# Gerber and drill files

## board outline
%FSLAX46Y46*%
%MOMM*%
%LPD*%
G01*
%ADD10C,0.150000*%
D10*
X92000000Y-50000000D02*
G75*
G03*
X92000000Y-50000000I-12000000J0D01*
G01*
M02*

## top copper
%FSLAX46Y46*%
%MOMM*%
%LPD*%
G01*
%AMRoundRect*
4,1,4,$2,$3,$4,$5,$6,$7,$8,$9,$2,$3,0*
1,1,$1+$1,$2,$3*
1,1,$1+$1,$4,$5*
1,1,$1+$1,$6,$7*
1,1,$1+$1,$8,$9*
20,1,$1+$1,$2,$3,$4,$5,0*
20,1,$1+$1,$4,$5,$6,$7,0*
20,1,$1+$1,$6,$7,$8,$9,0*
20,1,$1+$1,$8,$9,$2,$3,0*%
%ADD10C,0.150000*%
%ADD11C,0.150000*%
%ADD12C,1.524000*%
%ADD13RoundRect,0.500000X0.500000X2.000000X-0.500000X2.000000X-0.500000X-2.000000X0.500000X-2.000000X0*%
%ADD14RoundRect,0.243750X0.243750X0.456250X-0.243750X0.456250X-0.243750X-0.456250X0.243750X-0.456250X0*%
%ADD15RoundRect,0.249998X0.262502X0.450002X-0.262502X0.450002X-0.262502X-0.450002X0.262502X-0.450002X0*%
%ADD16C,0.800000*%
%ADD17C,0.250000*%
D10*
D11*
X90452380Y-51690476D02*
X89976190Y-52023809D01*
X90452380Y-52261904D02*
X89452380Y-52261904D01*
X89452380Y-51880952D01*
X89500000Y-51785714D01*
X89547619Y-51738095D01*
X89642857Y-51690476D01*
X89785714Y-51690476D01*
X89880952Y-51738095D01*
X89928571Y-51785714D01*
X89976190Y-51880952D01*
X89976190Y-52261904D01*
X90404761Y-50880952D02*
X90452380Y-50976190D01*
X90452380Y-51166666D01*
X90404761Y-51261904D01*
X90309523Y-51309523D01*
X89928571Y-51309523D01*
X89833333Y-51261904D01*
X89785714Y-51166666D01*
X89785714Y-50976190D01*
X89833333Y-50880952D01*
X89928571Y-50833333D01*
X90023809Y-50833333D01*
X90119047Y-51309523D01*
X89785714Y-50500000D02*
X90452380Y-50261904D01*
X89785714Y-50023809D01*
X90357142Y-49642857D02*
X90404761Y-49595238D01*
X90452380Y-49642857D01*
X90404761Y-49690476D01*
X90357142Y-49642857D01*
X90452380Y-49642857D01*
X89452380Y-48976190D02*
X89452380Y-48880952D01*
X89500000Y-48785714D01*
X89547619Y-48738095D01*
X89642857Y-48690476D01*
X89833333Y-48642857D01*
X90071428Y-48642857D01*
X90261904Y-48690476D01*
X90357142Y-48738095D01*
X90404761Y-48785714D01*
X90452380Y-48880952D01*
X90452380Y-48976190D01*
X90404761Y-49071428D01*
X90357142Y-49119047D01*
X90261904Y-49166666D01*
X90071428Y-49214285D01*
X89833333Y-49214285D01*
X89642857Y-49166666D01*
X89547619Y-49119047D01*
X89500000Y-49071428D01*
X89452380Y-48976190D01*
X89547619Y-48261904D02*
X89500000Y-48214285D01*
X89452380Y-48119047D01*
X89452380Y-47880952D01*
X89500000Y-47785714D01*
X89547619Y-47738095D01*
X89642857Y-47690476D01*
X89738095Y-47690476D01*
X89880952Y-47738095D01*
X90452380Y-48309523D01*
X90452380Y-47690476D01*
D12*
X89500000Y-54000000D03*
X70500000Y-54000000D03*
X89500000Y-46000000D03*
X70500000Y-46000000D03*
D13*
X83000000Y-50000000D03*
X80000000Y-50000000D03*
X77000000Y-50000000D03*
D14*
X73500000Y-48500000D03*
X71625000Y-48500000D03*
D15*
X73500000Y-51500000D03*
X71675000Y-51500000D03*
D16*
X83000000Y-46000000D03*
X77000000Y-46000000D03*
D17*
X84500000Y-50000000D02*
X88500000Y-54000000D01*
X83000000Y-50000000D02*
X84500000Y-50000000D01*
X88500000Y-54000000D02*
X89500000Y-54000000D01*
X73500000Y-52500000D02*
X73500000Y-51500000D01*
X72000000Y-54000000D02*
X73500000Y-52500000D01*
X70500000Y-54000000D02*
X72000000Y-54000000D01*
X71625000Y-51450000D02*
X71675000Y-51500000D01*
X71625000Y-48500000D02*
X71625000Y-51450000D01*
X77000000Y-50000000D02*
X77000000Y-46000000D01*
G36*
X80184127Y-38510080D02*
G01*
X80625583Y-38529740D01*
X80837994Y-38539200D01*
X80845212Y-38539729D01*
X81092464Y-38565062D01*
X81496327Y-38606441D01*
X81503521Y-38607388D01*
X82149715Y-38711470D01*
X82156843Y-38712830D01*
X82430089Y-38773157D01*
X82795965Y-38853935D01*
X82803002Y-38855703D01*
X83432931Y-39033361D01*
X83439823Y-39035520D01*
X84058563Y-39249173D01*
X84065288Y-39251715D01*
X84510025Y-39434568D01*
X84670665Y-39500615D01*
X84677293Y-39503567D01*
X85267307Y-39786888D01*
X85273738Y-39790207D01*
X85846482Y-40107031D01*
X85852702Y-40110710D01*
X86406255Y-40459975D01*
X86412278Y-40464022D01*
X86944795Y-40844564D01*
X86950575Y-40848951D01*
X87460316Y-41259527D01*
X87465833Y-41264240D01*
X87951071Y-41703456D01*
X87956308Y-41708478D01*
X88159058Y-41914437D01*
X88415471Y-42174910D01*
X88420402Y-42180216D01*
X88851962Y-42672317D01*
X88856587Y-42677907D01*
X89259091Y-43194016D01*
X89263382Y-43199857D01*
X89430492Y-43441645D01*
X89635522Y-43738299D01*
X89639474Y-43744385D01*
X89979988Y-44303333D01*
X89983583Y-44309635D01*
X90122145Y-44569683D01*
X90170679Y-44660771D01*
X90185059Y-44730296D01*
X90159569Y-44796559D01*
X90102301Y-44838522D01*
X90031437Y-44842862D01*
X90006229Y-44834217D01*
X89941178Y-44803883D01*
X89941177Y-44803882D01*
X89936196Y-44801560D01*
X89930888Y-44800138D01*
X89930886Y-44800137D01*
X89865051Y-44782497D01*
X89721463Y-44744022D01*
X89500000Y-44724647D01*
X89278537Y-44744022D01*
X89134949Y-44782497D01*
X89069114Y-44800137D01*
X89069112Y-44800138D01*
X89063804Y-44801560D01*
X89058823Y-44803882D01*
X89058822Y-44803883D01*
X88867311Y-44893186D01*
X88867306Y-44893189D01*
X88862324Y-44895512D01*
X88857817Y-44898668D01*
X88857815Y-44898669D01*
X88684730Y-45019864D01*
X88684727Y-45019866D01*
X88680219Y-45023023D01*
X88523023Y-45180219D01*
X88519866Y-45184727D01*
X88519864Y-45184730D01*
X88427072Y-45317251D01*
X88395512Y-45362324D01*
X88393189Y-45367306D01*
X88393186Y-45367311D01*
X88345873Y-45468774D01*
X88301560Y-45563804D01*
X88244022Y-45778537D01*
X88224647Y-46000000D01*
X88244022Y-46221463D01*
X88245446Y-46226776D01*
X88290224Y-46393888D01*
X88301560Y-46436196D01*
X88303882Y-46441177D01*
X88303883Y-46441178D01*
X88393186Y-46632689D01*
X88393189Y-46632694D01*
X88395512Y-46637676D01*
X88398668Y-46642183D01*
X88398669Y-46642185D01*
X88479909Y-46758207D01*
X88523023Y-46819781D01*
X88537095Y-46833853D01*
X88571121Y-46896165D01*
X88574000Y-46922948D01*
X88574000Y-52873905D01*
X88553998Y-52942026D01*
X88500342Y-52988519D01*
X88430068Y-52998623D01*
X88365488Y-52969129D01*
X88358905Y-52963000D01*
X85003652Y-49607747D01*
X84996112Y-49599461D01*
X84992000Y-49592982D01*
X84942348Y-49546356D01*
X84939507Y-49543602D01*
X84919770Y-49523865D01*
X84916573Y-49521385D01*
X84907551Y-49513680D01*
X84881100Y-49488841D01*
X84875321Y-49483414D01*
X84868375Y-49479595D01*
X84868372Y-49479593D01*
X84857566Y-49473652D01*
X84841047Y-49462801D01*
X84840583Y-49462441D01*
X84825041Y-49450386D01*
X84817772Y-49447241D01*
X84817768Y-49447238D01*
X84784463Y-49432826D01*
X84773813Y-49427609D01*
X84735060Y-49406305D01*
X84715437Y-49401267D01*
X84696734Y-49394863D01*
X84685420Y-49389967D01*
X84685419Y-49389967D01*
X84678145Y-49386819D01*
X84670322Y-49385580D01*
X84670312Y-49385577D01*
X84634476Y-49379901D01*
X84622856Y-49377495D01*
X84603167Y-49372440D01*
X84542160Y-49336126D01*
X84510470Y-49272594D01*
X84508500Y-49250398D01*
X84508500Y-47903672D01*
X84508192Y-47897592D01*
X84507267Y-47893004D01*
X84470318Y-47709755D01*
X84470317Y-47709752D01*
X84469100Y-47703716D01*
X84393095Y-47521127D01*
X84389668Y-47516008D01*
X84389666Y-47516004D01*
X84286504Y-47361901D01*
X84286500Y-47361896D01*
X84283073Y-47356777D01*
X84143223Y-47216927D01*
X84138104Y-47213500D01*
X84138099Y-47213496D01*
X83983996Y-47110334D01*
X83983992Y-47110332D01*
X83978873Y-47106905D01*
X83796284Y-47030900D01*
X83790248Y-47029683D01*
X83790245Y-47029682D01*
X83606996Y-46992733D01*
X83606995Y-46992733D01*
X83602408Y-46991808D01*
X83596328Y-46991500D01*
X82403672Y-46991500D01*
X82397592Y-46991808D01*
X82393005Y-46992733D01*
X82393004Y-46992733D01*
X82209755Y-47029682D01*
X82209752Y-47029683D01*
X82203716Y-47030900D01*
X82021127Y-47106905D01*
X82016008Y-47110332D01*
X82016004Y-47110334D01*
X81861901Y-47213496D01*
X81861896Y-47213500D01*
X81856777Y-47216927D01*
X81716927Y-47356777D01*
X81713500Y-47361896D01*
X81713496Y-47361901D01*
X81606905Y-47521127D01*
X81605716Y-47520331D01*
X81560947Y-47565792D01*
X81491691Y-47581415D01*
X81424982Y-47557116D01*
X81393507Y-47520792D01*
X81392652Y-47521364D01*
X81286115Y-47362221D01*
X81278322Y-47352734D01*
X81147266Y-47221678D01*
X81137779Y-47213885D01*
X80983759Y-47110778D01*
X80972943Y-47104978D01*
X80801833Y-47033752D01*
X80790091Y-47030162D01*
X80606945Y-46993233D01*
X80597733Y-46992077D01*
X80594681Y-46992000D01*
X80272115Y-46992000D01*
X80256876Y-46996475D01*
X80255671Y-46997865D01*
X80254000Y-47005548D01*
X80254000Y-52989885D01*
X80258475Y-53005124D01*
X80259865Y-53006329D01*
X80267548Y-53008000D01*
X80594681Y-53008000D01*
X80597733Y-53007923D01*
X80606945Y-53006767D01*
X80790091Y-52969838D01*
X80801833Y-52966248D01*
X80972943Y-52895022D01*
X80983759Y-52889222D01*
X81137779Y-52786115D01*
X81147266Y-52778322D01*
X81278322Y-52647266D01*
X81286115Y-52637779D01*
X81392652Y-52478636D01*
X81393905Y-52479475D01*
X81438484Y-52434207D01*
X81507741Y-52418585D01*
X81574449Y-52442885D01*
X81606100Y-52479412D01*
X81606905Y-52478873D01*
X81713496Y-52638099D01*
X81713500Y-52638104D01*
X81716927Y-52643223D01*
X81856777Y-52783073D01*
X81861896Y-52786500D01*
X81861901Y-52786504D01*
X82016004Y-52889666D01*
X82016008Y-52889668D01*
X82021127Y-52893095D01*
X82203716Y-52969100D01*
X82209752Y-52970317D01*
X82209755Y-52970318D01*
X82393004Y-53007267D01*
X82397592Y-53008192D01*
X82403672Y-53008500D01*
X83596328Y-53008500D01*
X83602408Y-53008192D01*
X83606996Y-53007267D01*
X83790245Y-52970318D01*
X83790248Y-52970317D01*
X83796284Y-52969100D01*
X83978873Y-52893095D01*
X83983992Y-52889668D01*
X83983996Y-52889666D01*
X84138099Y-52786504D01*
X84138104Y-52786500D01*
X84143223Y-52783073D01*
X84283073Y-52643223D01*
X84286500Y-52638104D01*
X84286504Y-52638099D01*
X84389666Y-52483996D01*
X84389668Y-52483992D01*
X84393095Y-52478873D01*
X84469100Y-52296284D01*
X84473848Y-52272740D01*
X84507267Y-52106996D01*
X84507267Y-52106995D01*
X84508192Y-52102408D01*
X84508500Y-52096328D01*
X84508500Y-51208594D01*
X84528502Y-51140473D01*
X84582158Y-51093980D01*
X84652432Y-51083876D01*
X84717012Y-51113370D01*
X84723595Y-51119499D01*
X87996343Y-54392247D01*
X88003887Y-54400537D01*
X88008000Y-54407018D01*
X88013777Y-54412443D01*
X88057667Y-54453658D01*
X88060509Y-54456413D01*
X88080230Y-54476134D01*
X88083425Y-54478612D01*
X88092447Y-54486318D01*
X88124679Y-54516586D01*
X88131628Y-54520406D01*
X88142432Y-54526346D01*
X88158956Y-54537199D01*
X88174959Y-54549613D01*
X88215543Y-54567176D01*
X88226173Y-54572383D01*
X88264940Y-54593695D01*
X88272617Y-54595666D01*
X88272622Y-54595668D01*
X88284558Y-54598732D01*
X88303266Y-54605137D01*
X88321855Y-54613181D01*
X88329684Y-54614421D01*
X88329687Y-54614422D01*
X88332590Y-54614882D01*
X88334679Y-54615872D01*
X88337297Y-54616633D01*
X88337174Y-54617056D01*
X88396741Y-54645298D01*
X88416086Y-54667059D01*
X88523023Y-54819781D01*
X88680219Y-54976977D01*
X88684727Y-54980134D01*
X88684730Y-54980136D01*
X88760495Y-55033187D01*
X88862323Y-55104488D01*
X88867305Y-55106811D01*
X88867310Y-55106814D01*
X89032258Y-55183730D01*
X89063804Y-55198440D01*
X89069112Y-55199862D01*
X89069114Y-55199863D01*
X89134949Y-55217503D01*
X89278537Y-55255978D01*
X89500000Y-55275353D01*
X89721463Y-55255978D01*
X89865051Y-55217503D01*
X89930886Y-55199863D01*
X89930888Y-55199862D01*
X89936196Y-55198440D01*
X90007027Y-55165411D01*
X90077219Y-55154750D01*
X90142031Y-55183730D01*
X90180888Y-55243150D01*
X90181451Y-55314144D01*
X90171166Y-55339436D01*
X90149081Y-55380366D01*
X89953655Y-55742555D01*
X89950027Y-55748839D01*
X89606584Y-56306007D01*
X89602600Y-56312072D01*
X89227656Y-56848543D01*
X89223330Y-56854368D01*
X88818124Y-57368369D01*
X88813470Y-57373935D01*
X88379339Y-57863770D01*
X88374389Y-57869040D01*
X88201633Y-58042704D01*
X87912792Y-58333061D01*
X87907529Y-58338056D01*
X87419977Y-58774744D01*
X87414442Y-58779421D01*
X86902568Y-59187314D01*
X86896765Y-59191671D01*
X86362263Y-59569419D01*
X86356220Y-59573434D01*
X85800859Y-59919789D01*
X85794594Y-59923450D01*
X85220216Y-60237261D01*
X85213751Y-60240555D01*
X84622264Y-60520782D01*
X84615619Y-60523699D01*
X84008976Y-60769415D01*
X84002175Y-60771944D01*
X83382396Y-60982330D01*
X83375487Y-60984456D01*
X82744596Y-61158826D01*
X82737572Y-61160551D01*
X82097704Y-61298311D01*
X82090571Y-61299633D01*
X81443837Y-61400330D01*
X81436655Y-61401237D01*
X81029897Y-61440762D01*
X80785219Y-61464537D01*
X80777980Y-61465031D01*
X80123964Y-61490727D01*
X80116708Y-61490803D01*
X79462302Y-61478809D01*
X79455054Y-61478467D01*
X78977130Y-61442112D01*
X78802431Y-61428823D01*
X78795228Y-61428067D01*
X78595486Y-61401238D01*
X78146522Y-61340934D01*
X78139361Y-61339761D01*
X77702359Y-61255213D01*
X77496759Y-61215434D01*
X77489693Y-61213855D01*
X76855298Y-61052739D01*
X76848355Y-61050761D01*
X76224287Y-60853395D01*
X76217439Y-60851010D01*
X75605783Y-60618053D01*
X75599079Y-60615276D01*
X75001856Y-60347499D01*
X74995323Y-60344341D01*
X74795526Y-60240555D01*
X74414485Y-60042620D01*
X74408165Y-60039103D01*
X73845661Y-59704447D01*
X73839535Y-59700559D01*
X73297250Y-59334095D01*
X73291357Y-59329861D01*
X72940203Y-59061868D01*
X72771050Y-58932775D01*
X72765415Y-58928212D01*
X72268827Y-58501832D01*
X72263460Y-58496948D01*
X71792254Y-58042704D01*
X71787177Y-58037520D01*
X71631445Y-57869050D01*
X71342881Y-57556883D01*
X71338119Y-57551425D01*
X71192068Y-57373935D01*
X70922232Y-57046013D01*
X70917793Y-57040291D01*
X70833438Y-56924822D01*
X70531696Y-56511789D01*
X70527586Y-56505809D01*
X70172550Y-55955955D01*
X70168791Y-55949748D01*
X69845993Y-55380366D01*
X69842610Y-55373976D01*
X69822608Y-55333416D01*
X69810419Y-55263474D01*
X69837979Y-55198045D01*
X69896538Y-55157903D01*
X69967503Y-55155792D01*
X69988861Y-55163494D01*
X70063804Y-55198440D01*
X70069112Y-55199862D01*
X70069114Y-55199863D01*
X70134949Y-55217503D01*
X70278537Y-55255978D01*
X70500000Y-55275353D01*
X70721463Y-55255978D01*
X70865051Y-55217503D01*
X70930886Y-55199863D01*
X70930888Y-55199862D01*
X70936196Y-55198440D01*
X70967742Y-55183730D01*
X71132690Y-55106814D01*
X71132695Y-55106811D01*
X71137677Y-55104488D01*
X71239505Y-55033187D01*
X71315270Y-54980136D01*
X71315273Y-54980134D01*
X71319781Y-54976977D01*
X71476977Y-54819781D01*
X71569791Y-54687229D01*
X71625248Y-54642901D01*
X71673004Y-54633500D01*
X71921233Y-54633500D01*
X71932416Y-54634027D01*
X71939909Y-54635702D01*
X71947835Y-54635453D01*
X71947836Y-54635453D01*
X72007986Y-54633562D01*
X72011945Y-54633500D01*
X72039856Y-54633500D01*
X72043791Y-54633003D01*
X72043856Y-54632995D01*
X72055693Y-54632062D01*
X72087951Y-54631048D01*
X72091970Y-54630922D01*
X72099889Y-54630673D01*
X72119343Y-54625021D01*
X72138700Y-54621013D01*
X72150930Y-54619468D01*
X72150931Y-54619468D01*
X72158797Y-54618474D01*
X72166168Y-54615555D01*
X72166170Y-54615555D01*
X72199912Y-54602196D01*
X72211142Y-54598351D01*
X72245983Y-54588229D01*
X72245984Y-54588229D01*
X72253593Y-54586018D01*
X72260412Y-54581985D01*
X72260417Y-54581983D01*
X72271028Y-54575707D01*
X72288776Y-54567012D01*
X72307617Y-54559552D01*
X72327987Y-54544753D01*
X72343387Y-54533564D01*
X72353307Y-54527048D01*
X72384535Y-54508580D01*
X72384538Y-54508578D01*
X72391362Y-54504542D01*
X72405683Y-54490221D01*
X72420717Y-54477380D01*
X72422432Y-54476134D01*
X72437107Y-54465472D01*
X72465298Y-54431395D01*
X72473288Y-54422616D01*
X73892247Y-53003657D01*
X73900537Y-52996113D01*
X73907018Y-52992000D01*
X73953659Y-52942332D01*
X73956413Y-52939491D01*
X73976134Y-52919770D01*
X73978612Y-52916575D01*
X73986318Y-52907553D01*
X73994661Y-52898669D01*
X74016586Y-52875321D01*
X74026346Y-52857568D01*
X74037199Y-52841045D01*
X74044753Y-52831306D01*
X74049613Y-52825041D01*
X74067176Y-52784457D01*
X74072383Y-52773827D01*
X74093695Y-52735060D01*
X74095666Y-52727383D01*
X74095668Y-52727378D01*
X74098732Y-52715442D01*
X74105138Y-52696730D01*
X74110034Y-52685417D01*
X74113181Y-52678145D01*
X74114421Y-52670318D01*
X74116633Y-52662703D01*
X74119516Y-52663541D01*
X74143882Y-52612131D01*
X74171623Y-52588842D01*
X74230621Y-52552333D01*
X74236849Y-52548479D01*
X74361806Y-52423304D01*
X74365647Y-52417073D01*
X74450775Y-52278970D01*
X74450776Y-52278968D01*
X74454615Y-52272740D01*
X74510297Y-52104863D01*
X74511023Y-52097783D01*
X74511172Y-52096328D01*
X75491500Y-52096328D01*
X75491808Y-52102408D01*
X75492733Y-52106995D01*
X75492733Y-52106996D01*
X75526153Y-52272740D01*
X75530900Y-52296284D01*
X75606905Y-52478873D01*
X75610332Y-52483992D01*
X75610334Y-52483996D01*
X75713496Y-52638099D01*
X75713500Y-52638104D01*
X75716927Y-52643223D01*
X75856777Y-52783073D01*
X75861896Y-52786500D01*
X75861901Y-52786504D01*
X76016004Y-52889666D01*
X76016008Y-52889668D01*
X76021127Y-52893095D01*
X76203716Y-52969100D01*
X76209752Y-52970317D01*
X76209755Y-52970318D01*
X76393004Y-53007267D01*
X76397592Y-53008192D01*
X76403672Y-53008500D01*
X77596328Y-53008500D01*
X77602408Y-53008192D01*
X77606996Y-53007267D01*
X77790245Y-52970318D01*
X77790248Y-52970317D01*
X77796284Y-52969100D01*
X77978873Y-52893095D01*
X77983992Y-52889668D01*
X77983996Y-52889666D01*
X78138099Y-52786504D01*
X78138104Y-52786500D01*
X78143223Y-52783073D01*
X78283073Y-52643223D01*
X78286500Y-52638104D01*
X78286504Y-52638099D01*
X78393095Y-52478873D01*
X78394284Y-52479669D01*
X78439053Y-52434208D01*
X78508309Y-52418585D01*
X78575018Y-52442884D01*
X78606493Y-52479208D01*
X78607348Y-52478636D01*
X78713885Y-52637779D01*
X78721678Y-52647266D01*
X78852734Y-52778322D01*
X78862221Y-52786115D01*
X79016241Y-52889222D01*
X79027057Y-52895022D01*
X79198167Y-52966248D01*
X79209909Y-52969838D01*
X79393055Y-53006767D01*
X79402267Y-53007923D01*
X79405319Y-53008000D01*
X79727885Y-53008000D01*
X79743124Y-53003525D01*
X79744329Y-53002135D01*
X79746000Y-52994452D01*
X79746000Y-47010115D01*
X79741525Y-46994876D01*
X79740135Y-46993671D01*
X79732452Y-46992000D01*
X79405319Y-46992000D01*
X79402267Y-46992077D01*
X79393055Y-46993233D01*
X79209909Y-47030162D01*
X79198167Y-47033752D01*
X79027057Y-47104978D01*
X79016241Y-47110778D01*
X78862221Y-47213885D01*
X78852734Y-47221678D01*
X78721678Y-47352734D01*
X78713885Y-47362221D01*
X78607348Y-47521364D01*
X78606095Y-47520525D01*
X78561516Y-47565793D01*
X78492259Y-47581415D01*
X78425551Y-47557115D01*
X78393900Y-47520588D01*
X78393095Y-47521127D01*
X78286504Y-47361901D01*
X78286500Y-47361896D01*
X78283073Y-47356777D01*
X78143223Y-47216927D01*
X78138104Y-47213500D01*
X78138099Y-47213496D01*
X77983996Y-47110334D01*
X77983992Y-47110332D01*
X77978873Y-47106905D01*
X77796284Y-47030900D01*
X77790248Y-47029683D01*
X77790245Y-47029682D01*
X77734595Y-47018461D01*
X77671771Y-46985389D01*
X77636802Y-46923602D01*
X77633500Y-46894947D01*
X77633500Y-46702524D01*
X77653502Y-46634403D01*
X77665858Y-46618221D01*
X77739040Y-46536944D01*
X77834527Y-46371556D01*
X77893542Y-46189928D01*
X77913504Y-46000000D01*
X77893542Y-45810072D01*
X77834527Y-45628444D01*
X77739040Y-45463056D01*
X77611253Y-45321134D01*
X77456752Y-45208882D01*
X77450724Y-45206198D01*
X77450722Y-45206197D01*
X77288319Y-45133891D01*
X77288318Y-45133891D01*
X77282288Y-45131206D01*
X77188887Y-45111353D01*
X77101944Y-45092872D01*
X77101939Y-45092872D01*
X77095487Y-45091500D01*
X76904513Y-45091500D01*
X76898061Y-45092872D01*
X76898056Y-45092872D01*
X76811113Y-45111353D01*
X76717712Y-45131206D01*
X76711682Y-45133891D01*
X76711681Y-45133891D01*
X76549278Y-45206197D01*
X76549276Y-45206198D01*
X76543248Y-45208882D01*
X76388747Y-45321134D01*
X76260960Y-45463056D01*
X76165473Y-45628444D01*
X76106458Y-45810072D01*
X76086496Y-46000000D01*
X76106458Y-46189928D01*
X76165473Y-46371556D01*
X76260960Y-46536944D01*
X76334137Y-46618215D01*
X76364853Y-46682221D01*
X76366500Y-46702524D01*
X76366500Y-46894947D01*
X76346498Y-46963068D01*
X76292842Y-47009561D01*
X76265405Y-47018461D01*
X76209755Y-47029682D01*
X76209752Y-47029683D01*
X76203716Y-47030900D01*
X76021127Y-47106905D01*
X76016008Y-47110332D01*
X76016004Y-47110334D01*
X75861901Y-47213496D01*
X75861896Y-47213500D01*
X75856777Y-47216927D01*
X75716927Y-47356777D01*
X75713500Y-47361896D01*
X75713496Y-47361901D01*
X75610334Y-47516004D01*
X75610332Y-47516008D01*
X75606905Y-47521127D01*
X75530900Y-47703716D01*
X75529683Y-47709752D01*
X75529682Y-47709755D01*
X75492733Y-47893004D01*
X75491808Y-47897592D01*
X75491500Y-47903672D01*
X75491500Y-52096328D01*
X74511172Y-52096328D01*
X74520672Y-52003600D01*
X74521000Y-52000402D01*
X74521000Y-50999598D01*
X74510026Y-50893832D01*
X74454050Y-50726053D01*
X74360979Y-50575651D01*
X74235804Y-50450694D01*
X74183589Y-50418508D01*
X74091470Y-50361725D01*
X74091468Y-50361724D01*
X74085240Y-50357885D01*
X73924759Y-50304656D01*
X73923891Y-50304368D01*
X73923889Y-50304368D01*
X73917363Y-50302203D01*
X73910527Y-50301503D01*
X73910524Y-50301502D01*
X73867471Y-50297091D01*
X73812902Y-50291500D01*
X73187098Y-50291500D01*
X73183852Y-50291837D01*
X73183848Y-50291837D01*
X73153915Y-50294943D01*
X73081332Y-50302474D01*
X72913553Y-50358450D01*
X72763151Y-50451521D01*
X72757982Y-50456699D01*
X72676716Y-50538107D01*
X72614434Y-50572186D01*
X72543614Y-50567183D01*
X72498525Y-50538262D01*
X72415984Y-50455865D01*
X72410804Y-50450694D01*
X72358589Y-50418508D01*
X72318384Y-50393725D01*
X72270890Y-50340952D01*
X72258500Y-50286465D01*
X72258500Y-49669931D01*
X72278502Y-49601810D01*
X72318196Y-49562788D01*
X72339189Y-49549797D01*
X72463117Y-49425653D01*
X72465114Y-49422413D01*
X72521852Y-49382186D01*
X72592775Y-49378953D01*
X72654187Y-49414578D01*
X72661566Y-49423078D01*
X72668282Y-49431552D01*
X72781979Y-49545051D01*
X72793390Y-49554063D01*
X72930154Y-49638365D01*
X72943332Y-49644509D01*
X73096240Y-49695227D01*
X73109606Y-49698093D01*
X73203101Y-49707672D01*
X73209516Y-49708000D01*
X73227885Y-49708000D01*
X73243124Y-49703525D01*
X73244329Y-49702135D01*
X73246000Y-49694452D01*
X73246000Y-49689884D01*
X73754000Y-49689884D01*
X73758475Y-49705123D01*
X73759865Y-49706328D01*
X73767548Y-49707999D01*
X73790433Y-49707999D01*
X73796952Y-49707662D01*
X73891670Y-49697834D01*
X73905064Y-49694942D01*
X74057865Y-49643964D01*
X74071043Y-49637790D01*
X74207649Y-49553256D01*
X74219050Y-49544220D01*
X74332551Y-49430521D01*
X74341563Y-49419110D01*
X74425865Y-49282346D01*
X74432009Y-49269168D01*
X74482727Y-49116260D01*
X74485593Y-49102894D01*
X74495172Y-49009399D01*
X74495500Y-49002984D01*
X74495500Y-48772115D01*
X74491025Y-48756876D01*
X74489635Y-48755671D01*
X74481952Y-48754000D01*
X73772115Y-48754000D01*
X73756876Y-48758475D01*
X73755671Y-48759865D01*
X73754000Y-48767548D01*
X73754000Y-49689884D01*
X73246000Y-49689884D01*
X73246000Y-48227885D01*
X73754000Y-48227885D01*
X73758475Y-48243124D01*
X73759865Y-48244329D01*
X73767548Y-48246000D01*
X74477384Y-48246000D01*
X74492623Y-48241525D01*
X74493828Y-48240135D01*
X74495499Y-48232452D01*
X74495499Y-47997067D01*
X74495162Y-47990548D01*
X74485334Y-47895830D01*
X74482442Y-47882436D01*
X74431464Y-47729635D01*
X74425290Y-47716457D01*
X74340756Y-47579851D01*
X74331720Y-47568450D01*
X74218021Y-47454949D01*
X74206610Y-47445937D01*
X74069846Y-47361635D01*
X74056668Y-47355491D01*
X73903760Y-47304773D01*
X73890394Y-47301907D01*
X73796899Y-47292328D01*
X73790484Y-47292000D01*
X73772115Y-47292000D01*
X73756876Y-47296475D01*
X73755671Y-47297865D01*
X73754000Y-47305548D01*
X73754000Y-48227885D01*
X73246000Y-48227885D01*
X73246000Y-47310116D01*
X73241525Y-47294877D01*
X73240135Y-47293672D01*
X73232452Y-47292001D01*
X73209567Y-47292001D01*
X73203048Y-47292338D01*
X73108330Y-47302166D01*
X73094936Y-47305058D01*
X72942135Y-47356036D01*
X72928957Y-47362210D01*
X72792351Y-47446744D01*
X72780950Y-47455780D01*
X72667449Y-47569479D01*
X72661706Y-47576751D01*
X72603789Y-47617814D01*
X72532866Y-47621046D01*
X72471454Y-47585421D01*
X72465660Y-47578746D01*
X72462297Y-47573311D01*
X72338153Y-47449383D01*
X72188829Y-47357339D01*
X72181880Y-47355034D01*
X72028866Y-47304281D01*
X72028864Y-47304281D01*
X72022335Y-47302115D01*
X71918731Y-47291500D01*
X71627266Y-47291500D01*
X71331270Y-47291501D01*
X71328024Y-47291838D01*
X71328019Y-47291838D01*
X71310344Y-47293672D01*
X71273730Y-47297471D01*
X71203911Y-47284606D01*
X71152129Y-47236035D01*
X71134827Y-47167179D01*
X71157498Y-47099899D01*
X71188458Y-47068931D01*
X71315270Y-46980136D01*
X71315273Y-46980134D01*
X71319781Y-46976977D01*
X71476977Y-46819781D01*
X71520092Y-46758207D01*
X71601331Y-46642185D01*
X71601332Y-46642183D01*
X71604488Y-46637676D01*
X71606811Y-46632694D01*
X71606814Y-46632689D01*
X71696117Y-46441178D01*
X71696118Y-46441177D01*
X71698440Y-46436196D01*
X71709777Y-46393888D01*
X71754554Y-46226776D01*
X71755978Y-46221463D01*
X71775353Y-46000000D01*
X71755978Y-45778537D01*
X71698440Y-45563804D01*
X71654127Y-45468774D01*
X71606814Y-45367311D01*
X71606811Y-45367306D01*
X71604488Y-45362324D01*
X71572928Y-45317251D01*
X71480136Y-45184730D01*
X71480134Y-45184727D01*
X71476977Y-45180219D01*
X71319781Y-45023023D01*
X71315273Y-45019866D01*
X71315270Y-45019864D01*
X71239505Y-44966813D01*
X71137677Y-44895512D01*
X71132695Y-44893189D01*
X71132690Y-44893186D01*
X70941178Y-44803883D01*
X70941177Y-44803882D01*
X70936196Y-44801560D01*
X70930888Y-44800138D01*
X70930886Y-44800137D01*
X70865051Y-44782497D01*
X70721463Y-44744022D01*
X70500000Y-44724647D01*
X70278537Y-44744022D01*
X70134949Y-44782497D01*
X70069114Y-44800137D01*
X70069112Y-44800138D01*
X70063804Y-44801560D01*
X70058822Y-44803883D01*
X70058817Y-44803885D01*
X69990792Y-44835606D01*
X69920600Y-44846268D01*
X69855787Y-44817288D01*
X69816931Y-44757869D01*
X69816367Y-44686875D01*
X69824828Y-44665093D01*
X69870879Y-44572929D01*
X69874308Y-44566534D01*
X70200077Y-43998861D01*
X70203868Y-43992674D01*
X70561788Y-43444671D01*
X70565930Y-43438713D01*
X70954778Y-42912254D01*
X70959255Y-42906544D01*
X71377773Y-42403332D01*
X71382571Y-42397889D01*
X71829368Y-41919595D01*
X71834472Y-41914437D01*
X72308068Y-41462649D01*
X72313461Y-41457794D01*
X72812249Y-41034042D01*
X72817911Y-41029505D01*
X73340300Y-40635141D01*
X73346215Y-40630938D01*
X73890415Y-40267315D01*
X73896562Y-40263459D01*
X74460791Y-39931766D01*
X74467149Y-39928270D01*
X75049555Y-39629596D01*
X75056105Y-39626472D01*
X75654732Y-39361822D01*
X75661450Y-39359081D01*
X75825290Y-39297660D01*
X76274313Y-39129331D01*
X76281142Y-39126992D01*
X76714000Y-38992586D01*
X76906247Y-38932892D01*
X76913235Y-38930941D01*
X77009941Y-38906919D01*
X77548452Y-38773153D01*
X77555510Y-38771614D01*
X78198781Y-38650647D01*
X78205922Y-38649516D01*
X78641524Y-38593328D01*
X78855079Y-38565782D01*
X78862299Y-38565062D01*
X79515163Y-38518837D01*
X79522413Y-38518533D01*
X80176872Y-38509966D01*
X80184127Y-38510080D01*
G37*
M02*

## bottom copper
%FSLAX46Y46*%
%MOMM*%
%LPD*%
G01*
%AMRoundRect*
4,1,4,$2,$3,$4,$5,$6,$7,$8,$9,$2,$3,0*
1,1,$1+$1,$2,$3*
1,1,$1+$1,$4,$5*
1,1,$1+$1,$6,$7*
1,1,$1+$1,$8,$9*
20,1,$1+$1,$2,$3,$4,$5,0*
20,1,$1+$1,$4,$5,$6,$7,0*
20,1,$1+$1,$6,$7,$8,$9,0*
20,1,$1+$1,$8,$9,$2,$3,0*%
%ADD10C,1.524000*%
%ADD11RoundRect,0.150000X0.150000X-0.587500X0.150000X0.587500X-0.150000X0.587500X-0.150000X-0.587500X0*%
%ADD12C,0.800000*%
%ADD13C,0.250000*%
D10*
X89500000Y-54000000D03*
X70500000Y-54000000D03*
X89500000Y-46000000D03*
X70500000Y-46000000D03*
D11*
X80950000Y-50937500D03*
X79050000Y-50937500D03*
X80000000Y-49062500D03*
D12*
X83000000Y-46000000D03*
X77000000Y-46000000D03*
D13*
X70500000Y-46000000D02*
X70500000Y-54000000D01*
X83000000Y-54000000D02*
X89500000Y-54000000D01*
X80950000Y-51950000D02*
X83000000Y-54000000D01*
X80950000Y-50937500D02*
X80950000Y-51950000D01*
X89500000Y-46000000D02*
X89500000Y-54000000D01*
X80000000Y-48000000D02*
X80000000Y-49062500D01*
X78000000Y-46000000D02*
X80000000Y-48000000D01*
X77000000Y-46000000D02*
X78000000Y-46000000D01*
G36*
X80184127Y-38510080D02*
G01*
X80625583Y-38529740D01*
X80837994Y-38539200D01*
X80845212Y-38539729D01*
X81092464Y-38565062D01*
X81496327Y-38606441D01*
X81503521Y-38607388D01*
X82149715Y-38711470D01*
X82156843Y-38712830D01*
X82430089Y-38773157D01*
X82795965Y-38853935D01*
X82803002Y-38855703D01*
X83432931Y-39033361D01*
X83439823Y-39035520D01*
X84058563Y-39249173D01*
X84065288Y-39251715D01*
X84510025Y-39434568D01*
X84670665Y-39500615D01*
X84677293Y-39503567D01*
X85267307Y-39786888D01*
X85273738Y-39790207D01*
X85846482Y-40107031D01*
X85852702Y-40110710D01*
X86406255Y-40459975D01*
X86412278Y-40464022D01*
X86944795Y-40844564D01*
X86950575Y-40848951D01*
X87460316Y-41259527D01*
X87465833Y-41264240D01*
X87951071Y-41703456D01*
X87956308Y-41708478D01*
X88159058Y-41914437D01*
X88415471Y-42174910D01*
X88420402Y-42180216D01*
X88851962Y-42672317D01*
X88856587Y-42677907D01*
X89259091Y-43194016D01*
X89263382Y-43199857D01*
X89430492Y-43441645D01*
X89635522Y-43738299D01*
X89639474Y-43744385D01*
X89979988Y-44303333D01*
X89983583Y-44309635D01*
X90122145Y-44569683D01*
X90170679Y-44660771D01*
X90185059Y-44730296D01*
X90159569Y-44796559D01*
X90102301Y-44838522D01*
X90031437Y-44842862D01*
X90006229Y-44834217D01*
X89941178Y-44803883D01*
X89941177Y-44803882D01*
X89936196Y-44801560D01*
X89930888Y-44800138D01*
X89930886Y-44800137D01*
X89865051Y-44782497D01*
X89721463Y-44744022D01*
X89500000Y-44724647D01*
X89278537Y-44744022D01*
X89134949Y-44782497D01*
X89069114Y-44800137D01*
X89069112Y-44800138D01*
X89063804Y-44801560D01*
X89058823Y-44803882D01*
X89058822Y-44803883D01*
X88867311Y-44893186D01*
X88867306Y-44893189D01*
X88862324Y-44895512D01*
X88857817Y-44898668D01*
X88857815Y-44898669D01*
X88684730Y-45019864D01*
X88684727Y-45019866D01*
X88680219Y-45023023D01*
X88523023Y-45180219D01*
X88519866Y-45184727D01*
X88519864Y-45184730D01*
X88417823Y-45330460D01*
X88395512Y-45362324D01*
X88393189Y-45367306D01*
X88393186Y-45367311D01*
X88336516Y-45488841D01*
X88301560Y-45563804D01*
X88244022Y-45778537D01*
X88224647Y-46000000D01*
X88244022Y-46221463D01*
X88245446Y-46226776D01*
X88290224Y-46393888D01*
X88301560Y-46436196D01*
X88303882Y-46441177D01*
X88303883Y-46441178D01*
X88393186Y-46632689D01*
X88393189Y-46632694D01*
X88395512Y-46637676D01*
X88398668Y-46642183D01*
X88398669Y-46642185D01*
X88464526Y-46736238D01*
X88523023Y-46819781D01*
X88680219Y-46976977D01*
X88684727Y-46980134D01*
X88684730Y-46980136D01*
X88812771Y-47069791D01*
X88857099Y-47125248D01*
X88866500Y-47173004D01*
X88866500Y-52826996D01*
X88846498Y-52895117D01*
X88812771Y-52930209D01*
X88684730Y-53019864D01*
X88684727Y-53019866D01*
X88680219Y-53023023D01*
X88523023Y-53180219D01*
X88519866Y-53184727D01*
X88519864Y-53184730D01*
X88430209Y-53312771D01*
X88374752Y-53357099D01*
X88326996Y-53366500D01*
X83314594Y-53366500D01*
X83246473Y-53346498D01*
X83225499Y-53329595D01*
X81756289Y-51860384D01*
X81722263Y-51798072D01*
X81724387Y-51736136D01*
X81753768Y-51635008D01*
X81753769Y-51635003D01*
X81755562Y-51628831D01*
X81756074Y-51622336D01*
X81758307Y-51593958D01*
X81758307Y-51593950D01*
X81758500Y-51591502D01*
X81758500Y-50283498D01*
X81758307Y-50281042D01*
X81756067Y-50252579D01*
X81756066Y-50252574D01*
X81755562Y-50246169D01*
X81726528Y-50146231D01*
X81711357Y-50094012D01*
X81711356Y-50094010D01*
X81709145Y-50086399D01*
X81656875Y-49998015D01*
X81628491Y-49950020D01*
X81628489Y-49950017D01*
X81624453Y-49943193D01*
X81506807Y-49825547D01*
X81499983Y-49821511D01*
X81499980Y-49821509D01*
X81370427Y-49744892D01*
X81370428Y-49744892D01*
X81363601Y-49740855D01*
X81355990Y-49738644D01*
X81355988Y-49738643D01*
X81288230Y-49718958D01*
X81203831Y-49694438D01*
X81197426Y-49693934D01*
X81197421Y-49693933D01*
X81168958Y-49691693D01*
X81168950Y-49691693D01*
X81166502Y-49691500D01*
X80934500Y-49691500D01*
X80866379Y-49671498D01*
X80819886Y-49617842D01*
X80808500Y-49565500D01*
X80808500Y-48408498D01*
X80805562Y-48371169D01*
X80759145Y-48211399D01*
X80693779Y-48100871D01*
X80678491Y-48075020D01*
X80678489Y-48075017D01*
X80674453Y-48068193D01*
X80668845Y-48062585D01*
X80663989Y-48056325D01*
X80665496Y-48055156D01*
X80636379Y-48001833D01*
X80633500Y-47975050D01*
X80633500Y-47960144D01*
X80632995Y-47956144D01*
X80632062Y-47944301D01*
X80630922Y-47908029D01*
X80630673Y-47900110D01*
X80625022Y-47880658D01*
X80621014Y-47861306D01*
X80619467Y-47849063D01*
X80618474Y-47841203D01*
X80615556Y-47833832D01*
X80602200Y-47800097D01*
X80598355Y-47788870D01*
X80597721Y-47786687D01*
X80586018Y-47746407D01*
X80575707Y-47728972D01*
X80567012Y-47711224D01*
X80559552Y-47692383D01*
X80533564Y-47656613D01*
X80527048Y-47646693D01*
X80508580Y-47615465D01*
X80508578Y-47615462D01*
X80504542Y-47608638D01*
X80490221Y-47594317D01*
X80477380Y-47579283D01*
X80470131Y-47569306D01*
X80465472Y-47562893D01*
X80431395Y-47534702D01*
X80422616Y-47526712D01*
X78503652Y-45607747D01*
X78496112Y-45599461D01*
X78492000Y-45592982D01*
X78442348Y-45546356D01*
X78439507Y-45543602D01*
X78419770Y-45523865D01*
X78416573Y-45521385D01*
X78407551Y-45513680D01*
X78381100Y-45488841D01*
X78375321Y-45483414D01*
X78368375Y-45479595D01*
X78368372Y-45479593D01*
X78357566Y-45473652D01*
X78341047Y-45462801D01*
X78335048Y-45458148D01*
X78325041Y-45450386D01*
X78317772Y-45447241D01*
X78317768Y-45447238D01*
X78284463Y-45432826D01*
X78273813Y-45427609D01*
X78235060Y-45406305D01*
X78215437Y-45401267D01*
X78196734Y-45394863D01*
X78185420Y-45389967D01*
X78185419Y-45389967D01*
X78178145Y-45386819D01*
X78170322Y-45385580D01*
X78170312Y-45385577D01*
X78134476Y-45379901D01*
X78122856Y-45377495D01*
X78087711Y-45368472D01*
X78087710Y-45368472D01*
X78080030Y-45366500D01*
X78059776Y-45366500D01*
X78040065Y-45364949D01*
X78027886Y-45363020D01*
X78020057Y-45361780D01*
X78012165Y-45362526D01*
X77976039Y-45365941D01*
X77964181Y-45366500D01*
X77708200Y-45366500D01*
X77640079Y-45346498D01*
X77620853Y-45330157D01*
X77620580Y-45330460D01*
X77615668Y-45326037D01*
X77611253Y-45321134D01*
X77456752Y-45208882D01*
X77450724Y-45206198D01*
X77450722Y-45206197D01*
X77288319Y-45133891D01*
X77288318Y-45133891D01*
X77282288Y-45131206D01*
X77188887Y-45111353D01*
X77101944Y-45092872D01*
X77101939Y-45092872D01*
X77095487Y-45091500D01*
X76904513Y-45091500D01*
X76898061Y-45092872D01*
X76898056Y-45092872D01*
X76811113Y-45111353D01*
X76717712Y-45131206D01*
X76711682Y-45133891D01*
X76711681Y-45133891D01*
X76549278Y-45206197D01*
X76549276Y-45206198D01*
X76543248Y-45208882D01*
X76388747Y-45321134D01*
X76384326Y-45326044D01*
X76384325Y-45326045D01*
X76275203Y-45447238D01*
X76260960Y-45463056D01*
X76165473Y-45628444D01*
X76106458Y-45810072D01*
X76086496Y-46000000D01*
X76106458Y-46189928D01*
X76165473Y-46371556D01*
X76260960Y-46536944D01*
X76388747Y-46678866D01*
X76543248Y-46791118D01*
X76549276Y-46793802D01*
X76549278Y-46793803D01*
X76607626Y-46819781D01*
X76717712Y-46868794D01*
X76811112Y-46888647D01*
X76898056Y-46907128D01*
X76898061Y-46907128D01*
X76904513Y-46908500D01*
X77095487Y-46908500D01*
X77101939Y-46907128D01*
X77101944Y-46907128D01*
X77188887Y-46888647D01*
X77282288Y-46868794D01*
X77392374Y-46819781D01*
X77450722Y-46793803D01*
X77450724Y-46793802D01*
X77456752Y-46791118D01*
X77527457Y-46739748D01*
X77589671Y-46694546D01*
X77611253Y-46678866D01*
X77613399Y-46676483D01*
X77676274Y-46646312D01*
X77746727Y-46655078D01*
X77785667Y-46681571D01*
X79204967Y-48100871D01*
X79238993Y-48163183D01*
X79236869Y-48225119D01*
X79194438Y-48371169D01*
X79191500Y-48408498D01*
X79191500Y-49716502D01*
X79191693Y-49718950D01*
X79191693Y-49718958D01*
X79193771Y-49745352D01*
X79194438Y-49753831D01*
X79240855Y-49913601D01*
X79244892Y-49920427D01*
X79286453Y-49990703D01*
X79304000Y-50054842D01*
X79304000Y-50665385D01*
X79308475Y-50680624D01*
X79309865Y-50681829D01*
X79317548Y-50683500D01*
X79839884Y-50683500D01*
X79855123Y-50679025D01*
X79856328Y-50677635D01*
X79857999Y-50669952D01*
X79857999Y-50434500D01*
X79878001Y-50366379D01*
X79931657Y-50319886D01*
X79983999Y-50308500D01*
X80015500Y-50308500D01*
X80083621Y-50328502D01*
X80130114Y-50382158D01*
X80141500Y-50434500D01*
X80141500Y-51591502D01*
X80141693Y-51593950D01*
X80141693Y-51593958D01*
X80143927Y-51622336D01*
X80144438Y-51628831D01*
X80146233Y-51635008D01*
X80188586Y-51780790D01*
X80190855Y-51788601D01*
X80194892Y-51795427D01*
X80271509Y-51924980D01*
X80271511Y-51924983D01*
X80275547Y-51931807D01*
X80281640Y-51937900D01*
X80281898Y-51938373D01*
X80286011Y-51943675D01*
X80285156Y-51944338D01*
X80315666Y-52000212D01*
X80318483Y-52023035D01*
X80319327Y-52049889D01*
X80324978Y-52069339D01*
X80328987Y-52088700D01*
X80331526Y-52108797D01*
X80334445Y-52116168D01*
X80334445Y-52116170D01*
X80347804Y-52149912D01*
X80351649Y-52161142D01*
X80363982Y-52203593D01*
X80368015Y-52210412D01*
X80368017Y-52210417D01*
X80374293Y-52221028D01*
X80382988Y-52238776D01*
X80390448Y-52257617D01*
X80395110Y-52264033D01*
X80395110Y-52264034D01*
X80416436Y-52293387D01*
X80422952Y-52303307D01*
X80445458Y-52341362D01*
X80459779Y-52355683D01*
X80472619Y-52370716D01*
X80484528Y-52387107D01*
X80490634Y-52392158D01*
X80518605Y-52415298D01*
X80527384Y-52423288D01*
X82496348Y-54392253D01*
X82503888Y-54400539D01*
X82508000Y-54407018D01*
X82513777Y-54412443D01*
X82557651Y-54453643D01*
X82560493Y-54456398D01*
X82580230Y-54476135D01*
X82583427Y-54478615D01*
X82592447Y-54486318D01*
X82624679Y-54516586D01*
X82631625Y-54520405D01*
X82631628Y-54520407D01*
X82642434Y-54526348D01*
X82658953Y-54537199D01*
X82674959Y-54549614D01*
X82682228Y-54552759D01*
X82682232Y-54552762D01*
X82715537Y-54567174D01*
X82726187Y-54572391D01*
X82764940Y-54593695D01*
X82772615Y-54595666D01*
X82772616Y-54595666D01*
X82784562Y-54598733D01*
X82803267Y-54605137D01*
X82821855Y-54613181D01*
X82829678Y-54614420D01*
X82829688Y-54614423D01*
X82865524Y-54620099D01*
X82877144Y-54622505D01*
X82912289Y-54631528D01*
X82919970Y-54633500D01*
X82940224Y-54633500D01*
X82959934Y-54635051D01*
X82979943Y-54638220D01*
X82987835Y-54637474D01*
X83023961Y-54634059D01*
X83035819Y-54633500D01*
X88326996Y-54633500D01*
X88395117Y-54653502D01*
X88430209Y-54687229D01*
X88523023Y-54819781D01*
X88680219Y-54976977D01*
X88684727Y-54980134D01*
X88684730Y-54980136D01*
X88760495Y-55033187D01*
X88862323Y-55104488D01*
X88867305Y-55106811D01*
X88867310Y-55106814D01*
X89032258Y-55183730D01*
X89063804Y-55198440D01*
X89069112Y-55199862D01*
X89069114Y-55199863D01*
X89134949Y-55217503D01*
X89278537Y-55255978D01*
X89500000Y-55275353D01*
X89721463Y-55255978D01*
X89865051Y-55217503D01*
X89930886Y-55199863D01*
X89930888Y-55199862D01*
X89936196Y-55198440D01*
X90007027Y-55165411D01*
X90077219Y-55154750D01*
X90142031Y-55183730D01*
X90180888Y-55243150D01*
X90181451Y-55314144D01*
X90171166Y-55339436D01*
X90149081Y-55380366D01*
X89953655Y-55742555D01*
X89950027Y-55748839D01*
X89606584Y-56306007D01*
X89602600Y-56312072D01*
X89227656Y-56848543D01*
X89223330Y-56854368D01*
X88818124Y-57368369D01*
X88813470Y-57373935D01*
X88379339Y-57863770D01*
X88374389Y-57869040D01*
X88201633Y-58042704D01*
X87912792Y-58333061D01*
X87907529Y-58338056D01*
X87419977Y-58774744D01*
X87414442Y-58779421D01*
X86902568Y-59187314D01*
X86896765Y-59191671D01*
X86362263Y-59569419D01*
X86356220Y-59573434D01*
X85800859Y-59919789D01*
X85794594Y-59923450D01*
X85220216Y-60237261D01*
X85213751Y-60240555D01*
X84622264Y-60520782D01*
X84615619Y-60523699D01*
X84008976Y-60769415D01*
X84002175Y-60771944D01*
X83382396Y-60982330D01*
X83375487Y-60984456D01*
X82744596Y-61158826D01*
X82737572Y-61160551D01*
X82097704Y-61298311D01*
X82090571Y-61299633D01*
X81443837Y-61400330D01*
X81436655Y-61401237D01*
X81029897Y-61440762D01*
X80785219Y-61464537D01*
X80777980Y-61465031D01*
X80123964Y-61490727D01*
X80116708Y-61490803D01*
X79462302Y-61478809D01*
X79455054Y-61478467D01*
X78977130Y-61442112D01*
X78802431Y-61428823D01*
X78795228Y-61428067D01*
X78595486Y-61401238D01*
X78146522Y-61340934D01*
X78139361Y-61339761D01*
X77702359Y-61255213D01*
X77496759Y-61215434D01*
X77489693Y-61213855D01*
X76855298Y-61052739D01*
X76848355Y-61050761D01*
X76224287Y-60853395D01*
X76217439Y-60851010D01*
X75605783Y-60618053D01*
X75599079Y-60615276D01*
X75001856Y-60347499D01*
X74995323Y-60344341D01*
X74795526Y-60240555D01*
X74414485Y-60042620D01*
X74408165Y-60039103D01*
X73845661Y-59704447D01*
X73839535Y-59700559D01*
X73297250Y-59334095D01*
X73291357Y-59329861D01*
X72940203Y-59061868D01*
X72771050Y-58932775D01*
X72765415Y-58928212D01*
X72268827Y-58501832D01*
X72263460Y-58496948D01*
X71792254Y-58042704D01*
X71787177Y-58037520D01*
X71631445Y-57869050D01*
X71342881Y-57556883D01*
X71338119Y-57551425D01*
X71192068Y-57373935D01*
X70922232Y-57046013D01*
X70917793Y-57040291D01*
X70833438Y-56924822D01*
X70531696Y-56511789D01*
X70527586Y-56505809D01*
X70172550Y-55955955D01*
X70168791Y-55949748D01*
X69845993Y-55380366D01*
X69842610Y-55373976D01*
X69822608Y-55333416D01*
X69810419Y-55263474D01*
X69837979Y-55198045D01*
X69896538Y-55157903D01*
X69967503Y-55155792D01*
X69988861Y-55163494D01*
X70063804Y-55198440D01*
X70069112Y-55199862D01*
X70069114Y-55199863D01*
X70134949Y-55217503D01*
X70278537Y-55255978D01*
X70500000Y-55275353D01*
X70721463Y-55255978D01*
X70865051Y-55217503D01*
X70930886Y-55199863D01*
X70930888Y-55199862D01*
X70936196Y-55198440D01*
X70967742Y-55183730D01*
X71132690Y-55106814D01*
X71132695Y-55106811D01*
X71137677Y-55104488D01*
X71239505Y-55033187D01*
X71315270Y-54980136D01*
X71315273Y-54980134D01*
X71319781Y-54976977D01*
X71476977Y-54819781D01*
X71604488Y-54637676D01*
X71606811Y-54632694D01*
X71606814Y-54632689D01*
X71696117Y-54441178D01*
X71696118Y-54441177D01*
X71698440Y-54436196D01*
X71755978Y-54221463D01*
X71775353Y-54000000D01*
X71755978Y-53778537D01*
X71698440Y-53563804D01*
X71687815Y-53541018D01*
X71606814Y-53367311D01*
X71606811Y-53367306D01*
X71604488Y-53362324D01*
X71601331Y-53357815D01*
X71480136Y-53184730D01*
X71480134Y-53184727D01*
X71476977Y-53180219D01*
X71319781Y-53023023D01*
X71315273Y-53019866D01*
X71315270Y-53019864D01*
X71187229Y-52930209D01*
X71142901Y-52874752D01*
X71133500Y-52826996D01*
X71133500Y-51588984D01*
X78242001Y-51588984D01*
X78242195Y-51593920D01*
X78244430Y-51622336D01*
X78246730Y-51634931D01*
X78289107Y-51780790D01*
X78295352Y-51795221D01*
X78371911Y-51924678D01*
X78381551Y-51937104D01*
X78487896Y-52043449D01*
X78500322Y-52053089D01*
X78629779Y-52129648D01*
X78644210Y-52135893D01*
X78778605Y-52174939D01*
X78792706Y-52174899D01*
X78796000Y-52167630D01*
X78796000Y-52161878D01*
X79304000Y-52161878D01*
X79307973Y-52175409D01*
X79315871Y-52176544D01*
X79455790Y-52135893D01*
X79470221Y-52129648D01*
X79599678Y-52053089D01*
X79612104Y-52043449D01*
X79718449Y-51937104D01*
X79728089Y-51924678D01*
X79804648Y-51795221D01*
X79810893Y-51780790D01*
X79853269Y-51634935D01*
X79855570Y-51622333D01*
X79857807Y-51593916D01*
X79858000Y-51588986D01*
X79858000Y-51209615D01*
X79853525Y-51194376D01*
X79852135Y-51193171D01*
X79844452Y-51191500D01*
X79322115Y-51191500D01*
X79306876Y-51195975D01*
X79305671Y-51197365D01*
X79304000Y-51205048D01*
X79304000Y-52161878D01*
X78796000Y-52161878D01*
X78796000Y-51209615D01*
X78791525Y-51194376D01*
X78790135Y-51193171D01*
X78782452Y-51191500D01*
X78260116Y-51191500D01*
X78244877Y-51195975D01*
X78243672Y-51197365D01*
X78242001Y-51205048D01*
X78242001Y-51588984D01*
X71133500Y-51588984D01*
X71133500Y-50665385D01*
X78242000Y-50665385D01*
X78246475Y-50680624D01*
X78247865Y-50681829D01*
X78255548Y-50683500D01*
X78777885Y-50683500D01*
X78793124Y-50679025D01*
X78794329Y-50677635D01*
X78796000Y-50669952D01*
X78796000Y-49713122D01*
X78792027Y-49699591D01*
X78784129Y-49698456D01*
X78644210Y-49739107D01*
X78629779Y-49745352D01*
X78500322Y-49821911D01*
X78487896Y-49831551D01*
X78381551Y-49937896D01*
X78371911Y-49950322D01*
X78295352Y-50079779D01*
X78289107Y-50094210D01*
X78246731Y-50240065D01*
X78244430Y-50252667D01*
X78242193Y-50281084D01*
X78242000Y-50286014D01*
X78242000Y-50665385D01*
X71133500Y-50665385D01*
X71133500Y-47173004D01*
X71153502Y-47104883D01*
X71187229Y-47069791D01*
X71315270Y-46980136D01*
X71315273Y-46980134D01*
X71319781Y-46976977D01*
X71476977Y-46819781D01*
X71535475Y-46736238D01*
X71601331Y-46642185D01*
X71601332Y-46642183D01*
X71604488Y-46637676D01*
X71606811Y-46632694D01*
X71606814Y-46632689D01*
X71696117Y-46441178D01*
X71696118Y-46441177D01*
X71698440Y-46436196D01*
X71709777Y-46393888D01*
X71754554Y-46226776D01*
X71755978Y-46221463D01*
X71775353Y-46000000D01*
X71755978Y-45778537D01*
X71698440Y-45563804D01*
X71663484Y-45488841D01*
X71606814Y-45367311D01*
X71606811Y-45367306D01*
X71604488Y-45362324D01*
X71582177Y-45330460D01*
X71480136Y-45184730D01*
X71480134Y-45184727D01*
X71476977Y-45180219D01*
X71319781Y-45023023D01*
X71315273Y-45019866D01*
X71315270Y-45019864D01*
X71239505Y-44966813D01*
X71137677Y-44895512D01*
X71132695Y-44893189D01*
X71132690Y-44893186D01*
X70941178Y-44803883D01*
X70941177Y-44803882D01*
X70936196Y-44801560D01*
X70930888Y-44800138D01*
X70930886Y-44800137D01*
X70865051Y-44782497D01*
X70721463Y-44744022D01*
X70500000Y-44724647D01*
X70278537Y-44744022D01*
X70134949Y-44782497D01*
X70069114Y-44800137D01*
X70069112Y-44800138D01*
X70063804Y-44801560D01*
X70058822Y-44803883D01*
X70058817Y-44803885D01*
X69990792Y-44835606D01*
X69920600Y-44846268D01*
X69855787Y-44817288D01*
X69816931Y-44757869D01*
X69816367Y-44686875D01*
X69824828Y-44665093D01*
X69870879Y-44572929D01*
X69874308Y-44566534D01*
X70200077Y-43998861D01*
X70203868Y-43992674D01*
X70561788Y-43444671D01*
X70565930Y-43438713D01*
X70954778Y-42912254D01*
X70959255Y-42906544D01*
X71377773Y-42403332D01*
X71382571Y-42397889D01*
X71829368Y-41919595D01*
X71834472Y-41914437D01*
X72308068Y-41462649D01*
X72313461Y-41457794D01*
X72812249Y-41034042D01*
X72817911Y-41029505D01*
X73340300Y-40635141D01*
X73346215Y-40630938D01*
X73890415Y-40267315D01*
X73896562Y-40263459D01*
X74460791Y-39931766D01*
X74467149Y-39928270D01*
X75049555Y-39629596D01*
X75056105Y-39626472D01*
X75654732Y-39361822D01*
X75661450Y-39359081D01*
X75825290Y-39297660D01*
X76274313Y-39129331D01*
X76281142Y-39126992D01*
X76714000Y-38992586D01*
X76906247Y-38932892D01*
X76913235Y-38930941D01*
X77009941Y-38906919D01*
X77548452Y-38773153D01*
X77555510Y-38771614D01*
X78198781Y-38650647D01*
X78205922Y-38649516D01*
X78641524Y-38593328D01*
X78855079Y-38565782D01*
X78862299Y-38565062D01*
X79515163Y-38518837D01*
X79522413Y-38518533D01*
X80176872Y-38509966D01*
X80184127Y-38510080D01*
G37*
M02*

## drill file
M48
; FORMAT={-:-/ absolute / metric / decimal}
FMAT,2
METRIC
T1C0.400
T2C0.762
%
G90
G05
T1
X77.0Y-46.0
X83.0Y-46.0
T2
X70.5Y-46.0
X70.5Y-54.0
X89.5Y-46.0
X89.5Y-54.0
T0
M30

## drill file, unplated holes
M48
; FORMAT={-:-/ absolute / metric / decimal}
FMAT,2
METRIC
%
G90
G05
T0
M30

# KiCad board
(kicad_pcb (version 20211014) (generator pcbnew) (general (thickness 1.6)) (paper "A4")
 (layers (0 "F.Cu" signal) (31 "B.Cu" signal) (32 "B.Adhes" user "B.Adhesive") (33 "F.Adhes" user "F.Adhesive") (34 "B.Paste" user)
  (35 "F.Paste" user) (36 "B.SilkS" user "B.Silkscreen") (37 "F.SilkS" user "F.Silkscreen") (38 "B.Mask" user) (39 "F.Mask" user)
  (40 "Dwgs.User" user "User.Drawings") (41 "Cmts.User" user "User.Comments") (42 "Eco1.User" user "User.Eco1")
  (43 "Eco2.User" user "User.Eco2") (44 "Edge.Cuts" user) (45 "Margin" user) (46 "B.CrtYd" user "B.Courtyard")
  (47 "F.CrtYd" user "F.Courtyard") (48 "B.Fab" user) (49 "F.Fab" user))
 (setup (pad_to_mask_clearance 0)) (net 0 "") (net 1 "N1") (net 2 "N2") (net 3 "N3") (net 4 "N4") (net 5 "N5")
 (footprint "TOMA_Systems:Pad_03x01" (layer "F.Cu") (at 80 50 180)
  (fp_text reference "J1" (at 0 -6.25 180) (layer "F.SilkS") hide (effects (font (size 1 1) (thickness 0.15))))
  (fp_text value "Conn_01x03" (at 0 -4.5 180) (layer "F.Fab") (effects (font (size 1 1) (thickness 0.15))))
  (pad "1" smd roundrect (at -3 0 180) (size 2 5) (layers "F.Cu" "F.Paste" "F.Mask") (roundrect_rratio 0.25) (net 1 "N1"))
  (pad "2" smd roundrect (at 0 0 180) (size 2 5) (layers "F.Cu" "F.Paste" "F.Mask") (roundrect_rratio 0.25) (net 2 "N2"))
  (pad "3" smd roundrect (at 3 0 180) (size 2 5) (layers "F.Cu" "F.Paste" "F.Mask") (roundrect_rratio 0.25) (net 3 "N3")))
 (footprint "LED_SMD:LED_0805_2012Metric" (layer "F.Cu") (at 72.5625 48.5 180)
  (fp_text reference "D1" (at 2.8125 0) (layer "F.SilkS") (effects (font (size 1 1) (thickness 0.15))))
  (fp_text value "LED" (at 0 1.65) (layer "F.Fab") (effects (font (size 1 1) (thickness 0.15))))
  (pad "1" smd roundrect locked (at -0.9375 0 180) (size 0.975 1.4) (layers "F.Cu" "F.Paste" "F.Mask") (roundrect_rratio 0.25) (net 2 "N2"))
  (pad "2" smd roundrect locked (at 0.9375 0 180) (size 0.975 1.4) (layers "F.Cu" "F.Paste" "F.Mask") (roundrect_rratio 0.25) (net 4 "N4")))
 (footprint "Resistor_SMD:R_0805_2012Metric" (layer "F.Cu") (at 72.5875 51.5 180)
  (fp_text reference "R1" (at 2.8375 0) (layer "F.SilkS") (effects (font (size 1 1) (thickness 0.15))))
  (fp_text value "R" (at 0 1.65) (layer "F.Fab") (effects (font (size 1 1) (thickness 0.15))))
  (pad "1" smd roundrect locked (at -0.9125 0 180) (size 1.025 1.4) (layers "F.Cu" "F.Paste" "F.Mask") (roundrect_rratio 0.2439004878)
   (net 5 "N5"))
  (pad "2" smd roundrect locked (at 0.9125 0 180) (size 1.025 1.4) (layers "F.Cu" "F.Paste" "F.Mask") (roundrect_rratio 0.2439004878)
   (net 4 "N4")))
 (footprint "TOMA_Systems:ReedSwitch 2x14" (layer "B.Cu") (at 80 54)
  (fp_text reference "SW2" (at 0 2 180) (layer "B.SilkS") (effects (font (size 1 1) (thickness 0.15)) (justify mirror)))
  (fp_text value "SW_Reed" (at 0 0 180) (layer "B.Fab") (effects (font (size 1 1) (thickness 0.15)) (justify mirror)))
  (pad "1" thru_hole circle (at 9.5 0) (size 1.524 1.524) (drill 0.762) (layers *.Cu *.Mask) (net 1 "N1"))
  (pad "2" thru_hole circle (at -9.5 0) (size 1.524 1.524) (drill 0.762) (layers *.Cu *.Mask) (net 5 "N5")))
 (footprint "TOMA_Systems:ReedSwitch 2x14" (layer "B.Cu") (at 80 46)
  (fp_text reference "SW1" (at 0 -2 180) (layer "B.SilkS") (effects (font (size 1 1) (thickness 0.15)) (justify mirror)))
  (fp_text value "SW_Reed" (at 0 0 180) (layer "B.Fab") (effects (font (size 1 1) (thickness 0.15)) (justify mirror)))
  (pad "1" thru_hole circle (at 9.5 0) (size 1.524 1.524) (drill 0.762) (layers *.Cu *.Mask) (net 1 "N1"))
  (pad "2" thru_hole circle (at -9.5 0) (size 1.524 1.524) (drill 0.762) (layers *.Cu *.Mask) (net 5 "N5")))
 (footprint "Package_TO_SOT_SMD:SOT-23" (layer "B.Cu") (at 80 50 90)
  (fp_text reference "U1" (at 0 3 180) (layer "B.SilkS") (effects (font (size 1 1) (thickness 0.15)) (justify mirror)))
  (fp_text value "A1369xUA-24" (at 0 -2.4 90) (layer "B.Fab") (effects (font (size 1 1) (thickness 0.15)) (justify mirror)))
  (pad "1" smd roundrect (at -0.9375 0.95 90) (size 1.475 0.6) (layers "B.Cu" "B.Paste" "B.Mask") (roundrect_rratio 0.25) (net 1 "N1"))
  (pad "2" smd roundrect (at -0.9375 -0.95 90) (size 1.475 0.6) (layers "B.Cu" "B.Paste" "B.Mask") (roundrect_rratio 0.25) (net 2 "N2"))
  (pad "3" smd roundrect (at 0.9375 0 90) (size 1.475 0.6) (layers "B.Cu" "B.Paste" "B.Mask") (roundrect_rratio 0.25) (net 3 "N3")))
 (gr_circle (center 80 50) (end 92 50) (layer "Edge.Cuts") (width 0.15) (fill none))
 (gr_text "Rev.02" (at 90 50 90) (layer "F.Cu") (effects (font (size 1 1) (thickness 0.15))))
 (via (at 83 46) (size 0.8) (drill 0.4) (layers "F.Cu" "B.Cu") (free) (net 2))
 (segment (start 71.625 51.45) (end 71.675 51.5) (width 0.25) (layer "F.Cu") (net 4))
 (segment (start 71.625 48.5) (end 71.625 51.45) (width 0.25) (layer "F.Cu") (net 4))
 (segment (start 70.5 54) (end 72 54) (width 0.25) (layer "F.Cu") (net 5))
 (segment (start 73.5 52.5) (end 73.5 51.5) (width 0.25) (layer "F.Cu") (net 5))
 (segment (start 72 54) (end 73.5 52.5) (width 0.25) (layer "F.Cu") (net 5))
 (segment (start 70.5 46) (end 70.5 54) (width 0.25) (layer "B.Cu") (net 5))
 (segment (start 83 50) (end 84.5 50) (width 0.25) (layer "F.Cu") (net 1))
 (segment (start 84.5 50) (end 88.5 54) (width 0.25) (layer "F.Cu") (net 1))
 (segment (start 88.5 54) (end 89.5 54) (width 0.25) (layer "F.Cu") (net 1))
 (segment (start 80.95 51.95) (end 83 54) (width 0.25) (layer "B.Cu") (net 1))
 (segment (start 89.5 46) (end 89.5 54) (width 0.25) (layer "B.Cu") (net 1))
 (segment (start 80.95 50.9375) (end 80.95 51.95) (width 0.25) (layer "B.Cu") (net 1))
 (segment (start 83 54) (end 89.5 54) (width 0.25) (layer "B.Cu") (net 1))
 (segment (start 77 50) (end 77 46) (width 0.25) (layer "F.Cu") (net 3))
 (via (at 77 46) (size 0.8) (drill 0.4) (layers "F.Cu" "B.Cu") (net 3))
 (segment (start 80 48) (end 80 49.0625) (width 0.25) (layer "B.Cu") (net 3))
 (segment (start 78 46) (end 80 48) (width 0.25) (layer "B.Cu") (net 3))
 (segment (start 77 46) (end 78 46) (width 0.25) (layer "B.Cu") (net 3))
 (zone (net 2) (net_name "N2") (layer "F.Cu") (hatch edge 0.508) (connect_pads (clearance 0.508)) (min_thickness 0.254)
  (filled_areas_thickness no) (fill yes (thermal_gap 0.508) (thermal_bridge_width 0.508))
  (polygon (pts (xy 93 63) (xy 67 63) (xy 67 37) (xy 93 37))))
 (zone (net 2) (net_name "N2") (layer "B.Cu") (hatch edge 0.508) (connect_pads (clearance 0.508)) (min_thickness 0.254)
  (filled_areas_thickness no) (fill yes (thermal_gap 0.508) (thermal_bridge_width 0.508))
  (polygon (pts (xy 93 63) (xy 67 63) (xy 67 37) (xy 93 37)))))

